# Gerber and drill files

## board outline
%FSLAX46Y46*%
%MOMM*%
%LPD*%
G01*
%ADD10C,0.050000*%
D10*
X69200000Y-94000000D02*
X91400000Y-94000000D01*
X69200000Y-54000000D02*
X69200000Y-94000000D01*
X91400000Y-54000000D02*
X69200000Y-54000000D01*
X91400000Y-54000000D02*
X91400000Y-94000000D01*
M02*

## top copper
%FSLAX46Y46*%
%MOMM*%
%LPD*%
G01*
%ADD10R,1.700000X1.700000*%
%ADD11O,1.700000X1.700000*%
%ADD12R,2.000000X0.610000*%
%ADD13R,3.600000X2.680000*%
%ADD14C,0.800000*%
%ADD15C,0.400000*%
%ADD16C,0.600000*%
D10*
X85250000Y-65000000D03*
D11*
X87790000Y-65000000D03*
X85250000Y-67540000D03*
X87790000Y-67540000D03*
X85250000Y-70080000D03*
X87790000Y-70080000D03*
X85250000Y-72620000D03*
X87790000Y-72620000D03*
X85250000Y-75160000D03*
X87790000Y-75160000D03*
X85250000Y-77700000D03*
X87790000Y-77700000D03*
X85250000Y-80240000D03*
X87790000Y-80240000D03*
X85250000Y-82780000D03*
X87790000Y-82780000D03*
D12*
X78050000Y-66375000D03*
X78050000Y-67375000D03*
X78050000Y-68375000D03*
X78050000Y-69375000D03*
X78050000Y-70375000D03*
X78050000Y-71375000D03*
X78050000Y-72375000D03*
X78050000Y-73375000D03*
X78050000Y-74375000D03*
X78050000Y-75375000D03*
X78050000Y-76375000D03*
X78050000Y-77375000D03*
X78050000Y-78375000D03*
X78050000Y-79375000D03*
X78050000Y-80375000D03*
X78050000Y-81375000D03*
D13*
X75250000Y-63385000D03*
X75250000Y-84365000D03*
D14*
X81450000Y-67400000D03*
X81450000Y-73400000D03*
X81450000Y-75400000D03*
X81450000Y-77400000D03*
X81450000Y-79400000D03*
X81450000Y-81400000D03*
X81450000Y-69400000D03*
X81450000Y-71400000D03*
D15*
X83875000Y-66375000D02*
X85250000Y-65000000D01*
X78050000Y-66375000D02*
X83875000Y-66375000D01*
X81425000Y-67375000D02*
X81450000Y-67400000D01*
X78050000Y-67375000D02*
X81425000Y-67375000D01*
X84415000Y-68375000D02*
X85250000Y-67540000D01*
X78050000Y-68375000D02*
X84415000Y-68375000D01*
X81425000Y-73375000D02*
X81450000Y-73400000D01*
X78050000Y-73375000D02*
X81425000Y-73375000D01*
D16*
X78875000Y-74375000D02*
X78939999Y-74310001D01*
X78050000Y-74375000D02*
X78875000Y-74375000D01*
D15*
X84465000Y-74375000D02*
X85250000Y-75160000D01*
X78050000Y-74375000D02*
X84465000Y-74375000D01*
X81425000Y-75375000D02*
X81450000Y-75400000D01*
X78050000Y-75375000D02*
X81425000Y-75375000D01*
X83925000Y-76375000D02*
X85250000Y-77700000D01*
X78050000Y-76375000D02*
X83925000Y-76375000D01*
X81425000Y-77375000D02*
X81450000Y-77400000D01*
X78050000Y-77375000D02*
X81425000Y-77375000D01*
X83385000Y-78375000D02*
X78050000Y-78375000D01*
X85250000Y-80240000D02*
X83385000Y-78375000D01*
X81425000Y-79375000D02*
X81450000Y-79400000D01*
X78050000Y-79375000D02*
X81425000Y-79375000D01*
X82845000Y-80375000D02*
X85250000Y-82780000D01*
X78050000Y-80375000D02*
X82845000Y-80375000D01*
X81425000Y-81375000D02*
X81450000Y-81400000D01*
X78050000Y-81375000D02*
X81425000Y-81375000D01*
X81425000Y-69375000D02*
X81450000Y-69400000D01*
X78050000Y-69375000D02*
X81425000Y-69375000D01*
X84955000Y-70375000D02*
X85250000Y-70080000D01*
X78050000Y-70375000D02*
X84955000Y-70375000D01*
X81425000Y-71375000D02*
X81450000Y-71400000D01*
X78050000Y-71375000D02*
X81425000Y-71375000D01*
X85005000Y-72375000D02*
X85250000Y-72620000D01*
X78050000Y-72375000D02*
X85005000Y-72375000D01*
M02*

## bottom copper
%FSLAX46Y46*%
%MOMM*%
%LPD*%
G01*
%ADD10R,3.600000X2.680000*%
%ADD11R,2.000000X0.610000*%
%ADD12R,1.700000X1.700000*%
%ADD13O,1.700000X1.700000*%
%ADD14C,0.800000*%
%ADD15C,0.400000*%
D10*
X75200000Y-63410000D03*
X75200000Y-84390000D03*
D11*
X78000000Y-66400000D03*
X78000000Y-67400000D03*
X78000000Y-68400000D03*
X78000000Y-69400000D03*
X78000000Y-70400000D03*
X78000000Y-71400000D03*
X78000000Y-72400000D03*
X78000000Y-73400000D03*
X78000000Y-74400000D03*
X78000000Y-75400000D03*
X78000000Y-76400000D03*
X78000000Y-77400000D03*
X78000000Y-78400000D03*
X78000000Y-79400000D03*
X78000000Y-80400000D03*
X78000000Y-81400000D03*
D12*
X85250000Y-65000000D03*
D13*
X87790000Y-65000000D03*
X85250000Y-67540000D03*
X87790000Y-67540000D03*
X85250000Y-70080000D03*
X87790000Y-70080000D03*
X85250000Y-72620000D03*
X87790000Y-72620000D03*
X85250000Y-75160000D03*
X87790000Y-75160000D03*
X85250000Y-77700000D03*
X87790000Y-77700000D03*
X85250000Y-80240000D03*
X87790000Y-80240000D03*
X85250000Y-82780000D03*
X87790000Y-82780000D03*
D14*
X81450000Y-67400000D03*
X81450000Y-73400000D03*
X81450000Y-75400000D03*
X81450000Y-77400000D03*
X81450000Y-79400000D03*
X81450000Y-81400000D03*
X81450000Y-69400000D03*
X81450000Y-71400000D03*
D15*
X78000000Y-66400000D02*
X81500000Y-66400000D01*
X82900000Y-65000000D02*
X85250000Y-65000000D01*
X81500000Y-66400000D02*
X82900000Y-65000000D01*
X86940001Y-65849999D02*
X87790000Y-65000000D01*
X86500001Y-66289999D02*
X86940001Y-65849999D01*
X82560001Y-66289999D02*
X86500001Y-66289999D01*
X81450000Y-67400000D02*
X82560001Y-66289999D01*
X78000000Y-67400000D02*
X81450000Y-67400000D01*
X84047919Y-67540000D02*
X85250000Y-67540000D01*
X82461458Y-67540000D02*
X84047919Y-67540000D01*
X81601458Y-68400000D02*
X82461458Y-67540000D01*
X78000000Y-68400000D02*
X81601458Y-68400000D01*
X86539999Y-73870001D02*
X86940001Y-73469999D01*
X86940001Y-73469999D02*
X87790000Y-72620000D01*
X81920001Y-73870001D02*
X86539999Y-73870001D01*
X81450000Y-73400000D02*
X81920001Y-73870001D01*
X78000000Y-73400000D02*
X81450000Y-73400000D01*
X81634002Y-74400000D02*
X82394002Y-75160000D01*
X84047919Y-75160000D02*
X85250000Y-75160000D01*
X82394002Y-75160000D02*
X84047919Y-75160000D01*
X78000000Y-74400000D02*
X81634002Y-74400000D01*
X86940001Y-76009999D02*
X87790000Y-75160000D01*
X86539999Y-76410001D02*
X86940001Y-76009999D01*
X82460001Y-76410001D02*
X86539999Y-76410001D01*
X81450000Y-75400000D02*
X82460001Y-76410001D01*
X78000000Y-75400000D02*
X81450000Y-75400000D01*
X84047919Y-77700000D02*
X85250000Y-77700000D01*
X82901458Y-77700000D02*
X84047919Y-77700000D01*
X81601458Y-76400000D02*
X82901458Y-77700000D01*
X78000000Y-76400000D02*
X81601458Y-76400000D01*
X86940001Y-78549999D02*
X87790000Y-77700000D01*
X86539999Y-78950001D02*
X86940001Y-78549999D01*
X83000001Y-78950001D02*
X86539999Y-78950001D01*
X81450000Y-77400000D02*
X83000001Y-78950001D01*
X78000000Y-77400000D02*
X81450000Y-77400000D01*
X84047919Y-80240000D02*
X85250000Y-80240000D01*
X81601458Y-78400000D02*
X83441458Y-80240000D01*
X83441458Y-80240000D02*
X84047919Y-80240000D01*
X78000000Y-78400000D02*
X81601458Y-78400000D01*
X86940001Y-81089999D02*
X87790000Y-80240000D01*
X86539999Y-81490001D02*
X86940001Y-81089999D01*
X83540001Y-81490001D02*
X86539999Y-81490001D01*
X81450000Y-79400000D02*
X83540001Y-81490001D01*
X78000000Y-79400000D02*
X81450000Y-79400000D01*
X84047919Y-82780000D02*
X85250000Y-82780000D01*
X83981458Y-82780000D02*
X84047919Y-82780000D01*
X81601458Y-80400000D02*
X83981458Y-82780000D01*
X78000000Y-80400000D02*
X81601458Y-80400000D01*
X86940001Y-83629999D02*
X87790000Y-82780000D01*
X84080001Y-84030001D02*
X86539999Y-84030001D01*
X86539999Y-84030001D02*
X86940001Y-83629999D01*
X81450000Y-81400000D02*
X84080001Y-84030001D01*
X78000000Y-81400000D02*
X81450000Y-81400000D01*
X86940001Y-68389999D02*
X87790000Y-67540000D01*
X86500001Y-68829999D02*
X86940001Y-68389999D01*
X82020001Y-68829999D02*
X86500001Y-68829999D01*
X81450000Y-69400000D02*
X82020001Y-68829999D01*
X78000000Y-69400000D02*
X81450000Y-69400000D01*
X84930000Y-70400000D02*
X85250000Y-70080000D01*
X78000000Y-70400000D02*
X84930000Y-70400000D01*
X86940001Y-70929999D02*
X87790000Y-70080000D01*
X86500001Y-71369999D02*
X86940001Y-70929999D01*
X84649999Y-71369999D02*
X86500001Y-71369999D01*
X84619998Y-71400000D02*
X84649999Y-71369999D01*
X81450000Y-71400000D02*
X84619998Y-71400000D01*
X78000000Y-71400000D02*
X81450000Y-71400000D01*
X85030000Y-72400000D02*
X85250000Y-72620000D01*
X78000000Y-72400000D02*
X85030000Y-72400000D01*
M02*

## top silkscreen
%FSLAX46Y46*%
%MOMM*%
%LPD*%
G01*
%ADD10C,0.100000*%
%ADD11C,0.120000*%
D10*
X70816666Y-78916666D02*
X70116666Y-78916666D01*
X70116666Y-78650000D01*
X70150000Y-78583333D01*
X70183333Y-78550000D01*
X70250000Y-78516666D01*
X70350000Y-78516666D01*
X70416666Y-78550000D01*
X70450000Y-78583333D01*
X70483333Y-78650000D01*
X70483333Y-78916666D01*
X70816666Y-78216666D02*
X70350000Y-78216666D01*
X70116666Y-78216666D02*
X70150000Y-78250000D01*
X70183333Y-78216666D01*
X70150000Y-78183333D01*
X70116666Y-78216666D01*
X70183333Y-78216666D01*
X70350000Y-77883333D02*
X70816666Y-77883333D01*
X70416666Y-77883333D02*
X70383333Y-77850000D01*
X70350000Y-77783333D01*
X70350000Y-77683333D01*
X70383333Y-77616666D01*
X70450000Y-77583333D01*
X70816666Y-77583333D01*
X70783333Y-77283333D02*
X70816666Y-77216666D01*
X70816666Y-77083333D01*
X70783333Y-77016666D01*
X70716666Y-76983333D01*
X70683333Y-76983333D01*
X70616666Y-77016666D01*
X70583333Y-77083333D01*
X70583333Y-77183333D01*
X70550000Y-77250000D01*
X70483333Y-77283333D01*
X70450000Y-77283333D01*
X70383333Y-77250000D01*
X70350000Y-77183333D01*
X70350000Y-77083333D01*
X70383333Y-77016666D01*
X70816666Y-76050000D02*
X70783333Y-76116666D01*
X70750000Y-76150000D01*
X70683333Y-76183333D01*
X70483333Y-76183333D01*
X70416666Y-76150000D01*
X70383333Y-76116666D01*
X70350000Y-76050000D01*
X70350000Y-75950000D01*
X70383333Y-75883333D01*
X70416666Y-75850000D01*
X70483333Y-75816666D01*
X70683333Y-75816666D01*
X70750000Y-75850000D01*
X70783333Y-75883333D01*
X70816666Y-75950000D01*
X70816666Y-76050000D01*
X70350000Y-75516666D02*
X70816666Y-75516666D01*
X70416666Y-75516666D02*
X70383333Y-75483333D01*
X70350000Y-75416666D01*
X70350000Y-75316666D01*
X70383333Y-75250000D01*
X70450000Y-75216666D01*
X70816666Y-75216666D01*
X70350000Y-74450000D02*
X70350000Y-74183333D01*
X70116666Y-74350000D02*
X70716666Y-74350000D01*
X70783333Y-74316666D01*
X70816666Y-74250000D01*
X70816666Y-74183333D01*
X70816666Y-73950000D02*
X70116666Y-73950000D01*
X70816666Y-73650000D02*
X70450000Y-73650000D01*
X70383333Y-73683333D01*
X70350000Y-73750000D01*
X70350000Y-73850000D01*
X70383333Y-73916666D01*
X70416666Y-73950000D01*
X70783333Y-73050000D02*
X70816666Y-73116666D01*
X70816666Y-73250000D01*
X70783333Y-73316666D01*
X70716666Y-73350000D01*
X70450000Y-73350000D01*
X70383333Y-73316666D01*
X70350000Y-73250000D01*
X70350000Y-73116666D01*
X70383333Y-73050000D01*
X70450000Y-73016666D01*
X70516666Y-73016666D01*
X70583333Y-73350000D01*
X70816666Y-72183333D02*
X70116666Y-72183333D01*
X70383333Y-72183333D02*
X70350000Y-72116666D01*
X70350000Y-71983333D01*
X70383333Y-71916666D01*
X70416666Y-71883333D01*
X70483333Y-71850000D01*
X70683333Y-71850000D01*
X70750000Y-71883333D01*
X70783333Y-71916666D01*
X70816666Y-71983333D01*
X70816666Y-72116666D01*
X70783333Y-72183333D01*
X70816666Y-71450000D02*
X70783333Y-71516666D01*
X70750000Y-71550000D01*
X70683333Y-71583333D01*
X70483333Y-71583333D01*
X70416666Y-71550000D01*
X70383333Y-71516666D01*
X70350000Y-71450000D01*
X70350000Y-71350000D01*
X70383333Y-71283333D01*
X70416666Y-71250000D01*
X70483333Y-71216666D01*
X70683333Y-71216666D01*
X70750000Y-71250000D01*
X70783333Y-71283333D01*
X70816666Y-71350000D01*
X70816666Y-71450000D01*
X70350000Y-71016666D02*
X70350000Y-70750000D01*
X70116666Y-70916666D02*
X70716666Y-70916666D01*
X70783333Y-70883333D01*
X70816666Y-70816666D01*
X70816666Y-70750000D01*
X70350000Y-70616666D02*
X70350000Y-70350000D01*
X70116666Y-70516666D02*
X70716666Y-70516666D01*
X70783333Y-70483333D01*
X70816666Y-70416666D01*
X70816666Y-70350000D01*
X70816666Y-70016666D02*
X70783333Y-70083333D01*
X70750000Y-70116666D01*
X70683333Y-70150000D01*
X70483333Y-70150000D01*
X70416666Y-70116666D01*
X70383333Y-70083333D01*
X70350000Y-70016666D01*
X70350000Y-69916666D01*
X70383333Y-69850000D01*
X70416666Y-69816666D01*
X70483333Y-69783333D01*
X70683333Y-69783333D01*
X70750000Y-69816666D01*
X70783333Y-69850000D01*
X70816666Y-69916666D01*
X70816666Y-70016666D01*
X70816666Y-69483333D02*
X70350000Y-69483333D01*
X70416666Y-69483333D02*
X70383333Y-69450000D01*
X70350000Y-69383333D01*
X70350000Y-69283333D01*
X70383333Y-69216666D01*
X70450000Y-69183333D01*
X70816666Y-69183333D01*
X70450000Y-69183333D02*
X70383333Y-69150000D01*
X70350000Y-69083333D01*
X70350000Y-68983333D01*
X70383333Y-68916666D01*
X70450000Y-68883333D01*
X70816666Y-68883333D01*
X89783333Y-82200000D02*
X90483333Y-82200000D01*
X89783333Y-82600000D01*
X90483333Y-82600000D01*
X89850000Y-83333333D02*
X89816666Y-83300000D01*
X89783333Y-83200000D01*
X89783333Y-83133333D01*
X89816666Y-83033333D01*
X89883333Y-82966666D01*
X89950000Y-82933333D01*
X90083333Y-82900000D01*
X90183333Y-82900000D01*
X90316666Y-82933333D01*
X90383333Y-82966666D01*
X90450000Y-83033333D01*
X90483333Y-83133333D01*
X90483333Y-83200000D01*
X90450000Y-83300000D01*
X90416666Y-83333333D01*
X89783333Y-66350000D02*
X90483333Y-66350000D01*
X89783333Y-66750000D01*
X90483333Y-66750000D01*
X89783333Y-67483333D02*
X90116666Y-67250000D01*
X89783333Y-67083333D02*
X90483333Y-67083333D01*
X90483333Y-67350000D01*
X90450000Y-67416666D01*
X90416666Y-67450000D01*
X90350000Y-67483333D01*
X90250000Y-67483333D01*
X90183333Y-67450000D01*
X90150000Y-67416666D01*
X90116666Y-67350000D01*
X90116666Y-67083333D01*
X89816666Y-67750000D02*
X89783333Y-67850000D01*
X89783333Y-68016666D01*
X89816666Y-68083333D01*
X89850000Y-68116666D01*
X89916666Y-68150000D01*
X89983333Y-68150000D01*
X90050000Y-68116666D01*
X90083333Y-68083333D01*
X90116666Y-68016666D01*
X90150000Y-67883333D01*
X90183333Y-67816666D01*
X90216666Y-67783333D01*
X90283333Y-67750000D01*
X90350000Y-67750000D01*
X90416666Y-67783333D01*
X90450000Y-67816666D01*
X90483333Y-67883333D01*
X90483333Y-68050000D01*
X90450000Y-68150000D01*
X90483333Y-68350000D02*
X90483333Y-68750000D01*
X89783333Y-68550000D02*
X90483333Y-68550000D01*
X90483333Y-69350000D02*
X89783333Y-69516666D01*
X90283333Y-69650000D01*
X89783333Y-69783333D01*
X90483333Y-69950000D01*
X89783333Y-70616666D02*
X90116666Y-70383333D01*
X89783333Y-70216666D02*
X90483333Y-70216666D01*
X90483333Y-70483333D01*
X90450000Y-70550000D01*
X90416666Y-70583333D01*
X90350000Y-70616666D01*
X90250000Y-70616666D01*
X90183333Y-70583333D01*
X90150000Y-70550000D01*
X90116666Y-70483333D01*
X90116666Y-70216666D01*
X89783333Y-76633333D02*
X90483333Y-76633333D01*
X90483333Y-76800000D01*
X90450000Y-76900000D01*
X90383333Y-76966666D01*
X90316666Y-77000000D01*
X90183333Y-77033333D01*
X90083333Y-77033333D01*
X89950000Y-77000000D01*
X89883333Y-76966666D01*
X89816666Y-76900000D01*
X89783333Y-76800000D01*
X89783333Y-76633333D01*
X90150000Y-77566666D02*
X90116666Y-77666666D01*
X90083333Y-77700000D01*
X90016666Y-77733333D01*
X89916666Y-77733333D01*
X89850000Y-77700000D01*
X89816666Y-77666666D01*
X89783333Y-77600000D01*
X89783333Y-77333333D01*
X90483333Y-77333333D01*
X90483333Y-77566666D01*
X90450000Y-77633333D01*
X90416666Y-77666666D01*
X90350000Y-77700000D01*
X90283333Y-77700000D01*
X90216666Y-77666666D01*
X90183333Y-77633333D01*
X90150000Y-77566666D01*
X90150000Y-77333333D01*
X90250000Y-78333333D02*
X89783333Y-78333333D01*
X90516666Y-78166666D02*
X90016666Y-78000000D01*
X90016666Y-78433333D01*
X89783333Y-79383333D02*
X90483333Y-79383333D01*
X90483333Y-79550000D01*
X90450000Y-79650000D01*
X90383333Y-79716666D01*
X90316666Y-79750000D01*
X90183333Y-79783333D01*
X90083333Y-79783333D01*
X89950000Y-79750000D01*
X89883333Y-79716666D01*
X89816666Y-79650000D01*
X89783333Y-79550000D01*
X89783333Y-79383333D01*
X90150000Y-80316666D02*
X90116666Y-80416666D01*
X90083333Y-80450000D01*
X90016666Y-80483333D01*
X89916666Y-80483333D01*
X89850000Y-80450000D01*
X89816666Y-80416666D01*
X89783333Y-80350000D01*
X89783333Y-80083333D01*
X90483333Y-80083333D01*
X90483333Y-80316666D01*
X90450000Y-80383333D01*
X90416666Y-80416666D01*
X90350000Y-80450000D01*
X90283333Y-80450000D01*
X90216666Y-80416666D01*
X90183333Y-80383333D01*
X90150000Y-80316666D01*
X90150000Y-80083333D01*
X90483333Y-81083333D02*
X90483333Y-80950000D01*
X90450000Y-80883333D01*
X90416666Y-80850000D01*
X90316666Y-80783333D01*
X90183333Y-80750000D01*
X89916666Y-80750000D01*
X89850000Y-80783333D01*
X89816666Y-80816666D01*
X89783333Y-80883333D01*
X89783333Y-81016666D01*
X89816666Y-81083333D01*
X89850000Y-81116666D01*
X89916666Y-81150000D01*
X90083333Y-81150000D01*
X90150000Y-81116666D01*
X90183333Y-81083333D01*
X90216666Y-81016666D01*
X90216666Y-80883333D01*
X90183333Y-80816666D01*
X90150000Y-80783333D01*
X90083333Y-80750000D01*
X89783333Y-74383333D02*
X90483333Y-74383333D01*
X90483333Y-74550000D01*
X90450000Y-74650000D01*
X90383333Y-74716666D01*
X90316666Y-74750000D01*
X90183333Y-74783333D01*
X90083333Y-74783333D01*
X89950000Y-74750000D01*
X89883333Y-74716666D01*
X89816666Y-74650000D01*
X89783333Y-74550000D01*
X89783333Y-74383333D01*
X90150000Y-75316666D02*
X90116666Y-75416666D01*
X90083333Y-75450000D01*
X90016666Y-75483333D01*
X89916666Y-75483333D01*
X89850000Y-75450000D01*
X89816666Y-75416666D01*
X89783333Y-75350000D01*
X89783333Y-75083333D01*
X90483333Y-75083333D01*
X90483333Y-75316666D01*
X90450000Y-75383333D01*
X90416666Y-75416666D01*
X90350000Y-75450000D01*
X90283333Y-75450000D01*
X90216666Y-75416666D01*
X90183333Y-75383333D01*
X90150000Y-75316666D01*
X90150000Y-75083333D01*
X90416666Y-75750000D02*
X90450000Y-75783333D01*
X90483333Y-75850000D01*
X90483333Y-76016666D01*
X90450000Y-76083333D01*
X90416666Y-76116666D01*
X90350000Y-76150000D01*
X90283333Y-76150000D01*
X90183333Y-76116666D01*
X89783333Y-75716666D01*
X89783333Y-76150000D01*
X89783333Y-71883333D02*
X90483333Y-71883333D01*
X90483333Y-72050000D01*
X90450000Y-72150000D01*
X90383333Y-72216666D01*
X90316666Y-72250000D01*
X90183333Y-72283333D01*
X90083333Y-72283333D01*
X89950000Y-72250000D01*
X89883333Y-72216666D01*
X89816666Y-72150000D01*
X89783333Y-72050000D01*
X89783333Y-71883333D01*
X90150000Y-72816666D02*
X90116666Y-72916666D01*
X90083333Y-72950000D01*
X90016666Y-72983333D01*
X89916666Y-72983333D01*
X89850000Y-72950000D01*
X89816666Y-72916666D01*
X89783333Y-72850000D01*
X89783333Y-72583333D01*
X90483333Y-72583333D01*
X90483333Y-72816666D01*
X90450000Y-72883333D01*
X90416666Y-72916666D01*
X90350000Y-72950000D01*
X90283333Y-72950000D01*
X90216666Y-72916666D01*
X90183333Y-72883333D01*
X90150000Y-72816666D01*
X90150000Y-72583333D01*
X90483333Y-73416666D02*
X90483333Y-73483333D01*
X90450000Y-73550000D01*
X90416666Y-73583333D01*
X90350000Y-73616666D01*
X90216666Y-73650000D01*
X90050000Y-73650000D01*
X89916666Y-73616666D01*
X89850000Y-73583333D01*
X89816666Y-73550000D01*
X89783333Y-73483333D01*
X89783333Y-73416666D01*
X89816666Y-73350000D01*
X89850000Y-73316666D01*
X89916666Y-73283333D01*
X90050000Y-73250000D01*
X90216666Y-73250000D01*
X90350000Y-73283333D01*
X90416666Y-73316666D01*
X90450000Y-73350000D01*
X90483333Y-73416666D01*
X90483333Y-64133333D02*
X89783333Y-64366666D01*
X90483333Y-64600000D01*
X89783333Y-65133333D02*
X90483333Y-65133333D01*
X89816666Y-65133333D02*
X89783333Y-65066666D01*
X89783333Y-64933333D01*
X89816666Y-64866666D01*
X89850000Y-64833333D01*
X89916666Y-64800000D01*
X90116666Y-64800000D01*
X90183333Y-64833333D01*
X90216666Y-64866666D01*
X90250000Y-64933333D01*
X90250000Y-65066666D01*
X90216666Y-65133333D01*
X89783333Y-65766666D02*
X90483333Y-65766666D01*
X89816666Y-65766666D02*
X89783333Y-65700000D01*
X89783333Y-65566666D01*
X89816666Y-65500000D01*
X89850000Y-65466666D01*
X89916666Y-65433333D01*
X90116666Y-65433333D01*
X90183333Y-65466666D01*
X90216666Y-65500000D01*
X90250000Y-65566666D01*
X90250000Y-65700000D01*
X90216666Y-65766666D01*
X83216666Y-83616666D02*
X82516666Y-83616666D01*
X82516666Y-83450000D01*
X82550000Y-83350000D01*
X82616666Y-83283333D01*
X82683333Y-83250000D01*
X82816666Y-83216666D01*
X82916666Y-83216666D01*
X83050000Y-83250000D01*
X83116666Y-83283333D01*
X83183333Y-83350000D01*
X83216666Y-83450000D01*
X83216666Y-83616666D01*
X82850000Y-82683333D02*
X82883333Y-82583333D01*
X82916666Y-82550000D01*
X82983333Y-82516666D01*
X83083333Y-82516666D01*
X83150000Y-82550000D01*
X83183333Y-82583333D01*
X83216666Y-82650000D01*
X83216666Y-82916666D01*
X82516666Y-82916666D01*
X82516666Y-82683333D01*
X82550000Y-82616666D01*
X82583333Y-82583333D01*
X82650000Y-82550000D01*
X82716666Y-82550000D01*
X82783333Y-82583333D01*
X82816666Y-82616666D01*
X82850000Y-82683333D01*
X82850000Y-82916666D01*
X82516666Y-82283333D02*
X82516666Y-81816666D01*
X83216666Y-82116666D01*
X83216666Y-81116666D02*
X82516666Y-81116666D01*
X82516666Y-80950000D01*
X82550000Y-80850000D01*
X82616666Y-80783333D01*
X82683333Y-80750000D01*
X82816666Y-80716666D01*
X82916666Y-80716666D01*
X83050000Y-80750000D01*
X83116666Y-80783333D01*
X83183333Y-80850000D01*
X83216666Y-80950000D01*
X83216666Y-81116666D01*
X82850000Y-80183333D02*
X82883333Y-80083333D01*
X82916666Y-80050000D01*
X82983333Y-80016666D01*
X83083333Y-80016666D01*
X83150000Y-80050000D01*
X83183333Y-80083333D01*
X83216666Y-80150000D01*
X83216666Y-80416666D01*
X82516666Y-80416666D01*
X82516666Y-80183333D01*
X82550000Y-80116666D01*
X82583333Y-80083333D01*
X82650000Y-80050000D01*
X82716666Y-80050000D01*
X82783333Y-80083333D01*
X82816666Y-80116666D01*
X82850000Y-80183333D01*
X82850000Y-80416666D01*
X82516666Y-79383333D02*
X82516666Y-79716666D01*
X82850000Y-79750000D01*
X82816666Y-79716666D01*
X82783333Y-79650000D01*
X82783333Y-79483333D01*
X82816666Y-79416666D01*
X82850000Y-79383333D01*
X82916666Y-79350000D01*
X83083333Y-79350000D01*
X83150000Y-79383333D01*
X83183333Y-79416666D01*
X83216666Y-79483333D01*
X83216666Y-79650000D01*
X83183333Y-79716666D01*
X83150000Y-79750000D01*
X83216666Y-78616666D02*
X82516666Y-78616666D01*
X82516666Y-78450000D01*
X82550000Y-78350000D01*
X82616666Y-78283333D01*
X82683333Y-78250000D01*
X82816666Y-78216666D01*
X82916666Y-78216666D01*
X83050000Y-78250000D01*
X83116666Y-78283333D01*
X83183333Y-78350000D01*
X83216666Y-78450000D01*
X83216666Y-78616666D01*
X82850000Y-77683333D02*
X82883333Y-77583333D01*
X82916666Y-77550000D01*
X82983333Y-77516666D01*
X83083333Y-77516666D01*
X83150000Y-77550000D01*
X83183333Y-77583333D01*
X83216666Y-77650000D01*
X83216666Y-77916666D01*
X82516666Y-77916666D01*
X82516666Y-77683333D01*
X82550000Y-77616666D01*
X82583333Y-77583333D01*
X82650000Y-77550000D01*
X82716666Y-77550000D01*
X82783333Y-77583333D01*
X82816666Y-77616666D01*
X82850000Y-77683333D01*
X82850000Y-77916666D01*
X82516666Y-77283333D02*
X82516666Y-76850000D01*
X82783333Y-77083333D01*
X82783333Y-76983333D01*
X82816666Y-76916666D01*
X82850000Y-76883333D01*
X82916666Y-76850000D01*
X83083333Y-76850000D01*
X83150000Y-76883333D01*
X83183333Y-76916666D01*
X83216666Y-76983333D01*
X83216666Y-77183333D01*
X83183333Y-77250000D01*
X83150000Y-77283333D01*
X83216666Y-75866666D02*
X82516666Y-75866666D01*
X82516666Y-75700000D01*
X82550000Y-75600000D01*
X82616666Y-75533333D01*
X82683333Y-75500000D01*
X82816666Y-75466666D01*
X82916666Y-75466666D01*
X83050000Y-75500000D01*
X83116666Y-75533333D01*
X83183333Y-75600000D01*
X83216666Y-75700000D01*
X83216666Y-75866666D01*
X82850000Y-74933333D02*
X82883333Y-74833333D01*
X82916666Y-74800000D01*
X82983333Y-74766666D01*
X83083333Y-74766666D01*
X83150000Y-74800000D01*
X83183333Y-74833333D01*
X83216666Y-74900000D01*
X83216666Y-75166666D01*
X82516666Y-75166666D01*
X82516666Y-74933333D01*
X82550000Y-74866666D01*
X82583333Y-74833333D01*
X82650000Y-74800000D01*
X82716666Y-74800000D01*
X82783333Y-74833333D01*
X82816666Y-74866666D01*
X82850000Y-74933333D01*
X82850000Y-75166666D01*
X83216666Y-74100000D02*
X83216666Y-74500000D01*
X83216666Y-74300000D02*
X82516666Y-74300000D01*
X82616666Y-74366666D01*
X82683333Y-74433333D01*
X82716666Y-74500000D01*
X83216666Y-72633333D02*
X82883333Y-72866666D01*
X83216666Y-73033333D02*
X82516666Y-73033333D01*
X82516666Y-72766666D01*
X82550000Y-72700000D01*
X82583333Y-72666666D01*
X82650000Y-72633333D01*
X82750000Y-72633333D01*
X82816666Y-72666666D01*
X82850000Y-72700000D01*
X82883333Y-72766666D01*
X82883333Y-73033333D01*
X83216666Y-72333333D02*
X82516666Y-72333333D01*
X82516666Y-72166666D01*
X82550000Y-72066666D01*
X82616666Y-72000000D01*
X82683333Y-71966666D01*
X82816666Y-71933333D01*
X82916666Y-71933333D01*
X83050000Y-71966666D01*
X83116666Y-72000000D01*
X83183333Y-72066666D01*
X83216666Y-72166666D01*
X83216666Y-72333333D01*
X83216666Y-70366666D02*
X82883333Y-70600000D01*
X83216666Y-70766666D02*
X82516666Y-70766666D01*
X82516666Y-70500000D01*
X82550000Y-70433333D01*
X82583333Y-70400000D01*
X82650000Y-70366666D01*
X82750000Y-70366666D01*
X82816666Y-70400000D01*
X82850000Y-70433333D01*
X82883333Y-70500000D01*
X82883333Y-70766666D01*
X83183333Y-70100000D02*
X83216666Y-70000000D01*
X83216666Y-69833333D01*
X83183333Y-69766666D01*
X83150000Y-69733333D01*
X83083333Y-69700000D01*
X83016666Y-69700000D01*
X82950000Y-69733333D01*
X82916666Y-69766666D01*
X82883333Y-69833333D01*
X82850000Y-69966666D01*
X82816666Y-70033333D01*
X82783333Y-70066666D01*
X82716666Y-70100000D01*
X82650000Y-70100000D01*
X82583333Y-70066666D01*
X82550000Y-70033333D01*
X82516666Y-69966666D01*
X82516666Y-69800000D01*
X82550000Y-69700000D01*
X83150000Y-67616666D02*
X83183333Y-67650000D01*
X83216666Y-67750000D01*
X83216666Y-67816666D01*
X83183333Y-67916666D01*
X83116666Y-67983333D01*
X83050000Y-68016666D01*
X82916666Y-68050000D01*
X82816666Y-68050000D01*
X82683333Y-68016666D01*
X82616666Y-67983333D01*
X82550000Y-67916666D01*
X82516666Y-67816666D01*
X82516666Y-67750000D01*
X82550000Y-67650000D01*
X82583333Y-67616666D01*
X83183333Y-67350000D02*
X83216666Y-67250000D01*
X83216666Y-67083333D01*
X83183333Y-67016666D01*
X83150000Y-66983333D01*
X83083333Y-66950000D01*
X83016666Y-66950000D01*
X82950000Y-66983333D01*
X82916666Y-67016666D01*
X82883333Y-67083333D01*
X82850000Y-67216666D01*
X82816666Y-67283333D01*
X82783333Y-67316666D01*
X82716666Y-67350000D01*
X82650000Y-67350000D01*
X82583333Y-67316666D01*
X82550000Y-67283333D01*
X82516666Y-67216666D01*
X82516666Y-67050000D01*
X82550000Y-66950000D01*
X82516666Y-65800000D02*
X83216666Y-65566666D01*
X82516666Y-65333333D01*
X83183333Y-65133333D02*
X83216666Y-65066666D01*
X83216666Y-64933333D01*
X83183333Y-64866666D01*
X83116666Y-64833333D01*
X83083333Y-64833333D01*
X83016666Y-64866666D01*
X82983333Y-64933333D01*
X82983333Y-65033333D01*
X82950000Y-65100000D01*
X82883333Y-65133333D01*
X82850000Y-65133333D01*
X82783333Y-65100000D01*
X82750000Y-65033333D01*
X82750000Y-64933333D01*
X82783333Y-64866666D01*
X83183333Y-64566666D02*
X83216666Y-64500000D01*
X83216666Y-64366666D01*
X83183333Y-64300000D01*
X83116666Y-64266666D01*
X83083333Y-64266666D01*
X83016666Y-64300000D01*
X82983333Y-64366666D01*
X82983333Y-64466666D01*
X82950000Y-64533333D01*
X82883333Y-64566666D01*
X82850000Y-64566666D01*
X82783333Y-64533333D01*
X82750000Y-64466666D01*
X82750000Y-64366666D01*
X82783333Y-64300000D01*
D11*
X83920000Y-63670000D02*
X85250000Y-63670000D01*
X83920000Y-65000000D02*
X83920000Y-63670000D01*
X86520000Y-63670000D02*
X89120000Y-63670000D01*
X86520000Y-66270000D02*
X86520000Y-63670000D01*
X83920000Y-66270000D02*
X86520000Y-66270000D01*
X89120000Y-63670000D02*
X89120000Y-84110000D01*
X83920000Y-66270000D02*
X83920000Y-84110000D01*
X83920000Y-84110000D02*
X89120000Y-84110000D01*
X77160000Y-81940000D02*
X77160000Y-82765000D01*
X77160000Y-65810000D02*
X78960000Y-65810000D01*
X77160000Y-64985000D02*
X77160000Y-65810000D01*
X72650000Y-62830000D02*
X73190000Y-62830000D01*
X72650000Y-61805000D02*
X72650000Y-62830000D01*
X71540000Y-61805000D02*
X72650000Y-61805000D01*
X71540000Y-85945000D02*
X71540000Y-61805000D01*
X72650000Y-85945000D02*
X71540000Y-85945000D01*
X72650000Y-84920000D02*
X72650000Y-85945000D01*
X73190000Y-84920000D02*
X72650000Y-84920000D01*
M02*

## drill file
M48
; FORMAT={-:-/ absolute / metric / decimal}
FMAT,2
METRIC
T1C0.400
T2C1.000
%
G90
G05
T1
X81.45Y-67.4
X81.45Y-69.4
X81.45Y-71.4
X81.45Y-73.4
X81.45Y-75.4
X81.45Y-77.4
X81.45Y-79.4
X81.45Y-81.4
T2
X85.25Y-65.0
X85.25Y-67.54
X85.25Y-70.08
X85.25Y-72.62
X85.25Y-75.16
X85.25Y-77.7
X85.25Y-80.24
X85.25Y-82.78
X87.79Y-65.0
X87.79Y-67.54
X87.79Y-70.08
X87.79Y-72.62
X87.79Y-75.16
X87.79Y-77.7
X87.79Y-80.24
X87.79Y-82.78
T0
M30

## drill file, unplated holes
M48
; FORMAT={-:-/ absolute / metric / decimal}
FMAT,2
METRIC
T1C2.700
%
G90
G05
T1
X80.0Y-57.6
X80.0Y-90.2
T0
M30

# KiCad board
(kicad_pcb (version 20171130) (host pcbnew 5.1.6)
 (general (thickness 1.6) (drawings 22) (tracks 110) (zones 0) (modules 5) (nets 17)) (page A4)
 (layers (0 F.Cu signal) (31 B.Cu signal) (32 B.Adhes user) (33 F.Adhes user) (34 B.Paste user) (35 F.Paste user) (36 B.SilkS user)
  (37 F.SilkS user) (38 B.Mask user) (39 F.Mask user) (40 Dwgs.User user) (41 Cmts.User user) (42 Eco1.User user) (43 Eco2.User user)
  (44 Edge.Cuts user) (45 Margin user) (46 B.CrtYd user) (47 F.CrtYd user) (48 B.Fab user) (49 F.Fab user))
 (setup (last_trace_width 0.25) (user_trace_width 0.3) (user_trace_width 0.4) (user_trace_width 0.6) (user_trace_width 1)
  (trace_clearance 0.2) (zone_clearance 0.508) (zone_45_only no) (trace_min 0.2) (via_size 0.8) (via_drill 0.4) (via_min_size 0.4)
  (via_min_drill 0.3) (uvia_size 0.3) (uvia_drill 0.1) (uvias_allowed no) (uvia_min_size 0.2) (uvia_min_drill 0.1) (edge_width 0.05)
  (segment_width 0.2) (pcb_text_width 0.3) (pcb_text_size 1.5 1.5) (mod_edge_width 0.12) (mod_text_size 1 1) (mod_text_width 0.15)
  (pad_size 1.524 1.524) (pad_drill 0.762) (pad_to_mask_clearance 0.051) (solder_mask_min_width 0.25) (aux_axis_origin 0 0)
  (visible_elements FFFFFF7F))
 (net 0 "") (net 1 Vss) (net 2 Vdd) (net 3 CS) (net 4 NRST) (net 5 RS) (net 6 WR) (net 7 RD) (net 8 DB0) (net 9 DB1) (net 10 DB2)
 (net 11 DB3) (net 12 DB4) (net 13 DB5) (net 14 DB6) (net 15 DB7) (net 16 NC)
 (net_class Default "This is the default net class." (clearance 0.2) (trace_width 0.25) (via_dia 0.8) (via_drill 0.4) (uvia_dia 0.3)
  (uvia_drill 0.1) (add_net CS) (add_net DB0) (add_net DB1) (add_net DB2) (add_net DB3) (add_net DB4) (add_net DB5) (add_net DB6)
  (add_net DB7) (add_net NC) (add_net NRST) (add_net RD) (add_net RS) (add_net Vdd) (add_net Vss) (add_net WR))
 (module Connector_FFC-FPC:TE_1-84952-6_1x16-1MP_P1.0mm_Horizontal (layer B.Cu) (at 76.2 73.9 90)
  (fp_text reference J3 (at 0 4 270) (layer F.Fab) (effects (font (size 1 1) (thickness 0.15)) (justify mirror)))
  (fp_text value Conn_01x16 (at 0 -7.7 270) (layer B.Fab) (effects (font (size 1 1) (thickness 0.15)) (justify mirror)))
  (pad MP smd rect (at 10.49 -1 90) (size 2.68 3.6) (layers B.Cu B.Paste B.Mask))
  (pad MP smd rect (at -10.49 -1 90) (size 2.68 3.6) (layers B.Cu B.Paste B.Mask))
  (pad 16 smd rect (at 7.5 1.8 90) (size 0.61 2) (layers B.Cu B.Paste B.Mask) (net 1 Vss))
  (pad 15 smd rect (at 6.5 1.8 90) (size 0.61 2) (layers B.Cu B.Paste B.Mask) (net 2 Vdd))
  (pad 14 smd rect (at 5.5 1.8 90) (size 0.61 2) (layers B.Cu B.Paste B.Mask) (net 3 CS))
  (pad 13 smd rect (at 4.5 1.8 90) (size 0.61 2) (layers B.Cu B.Paste B.Mask) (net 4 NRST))
  (pad 12 smd rect (at 3.5 1.8 90) (size 0.61 2) (layers B.Cu B.Paste B.Mask) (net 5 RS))
  (pad 11 smd rect (at 2.5 1.8 90) (size 0.61 2) (layers B.Cu B.Paste B.Mask) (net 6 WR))
  (pad 10 smd rect (at 1.5 1.8 90) (size 0.61 2) (layers B.Cu B.Paste B.Mask) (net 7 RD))
  (pad 9 smd rect (at 0.5 1.8 90) (size 0.61 2) (layers B.Cu B.Paste B.Mask) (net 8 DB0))
  (pad 8 smd rect (at -0.5 1.8 90) (size 0.61 2) (layers B.Cu B.Paste B.Mask) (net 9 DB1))
  (pad 7 smd rect (at -1.5 1.8 90) (size 0.61 2) (layers B.Cu B.Paste B.Mask) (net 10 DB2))
  (pad 6 smd rect (at -2.5 1.8 90) (size 0.61 2) (layers B.Cu B.Paste B.Mask) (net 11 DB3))
  (pad 5 smd rect (at -3.5 1.8 90) (size 0.61 2) (layers B.Cu B.Paste B.Mask) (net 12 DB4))
  (pad 4 smd rect (at -4.5 1.8 90) (size 0.61 2) (layers B.Cu B.Paste B.Mask) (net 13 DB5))
  (pad 3 smd rect (at -5.5 1.8 90) (size 0.61 2) (layers B.Cu B.Paste B.Mask) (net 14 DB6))
  (pad 2 smd rect (at -6.5 1.8 90) (size 0.61 2) (layers B.Cu B.Paste B.Mask) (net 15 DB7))
  (pad 1 smd rect (at -7.5 1.8 90) (size 0.61 2) (layers B.Cu B.Paste B.Mask) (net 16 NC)))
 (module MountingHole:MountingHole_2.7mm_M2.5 (layer F.Cu) (at 80 90.2)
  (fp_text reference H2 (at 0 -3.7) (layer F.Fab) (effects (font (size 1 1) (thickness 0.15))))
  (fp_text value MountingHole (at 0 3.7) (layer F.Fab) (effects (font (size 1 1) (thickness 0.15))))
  (pad 1 np_thru_hole circle (at 0 0) (size 2.7 2.7) (drill 2.7) (layers *.Cu *.Mask)))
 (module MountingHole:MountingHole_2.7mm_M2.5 (layer F.Cu) (at 80 57.6)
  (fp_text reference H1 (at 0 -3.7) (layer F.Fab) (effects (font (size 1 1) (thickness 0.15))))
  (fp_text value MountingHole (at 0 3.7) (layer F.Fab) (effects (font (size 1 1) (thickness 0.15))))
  (pad 1 np_thru_hole circle (at 0 0) (size 2.7 2.7) (drill 2.7) (layers *.Cu *.Mask)))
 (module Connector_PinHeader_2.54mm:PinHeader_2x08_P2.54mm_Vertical (layer F.Cu) (at 85.25 65)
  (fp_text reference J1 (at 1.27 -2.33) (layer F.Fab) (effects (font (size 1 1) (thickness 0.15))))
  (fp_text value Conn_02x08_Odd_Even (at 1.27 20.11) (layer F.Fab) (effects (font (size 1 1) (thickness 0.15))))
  (fp_line (start -1.33 -1.33) (end 0 -1.33) (layer F.SilkS) (width 0.12))
  (fp_line (start -1.33 0) (end -1.33 -1.33) (layer F.SilkS) (width 0.12))
  (fp_line (start 1.27 -1.33) (end 3.87 -1.33) (layer F.SilkS) (width 0.12))
  (fp_line (start 1.27 1.27) (end 1.27 -1.33) (layer F.SilkS) (width 0.12))
  (fp_line (start -1.33 1.27) (end 1.27 1.27) (layer F.SilkS) (width 0.12))
  (fp_line (start 3.87 -1.33) (end 3.87 19.11) (layer F.SilkS) (width 0.12))
  (fp_line (start -1.33 1.27) (end -1.33 19.11) (layer F.SilkS) (width 0.12))
  (fp_line (start -1.33 19.11) (end 3.87 19.11) (layer F.SilkS) (width 0.12))
  (pad 1 thru_hole rect (at 0 0) (size 1.7 1.7) (drill 1) (layers *.Cu *.Mask) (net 1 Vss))
  (pad 2 thru_hole oval (at 2.54 0) (size 1.7 1.7) (drill 1) (layers *.Cu *.Mask) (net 2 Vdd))
  (pad 3 thru_hole oval (at 0 2.54) (size 1.7 1.7) (drill 1) (layers *.Cu *.Mask) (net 3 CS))
  (pad 4 thru_hole oval (at 2.54 2.54) (size 1.7 1.7) (drill 1) (layers *.Cu *.Mask) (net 4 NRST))
  (pad 5 thru_hole oval (at 0 5.08) (size 1.7 1.7) (drill 1) (layers *.Cu *.Mask) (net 5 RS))
  (pad 6 thru_hole oval (at 2.54 5.08) (size 1.7 1.7) (drill 1) (layers *.Cu *.Mask) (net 6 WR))
  (pad 7 thru_hole oval (at 0 7.62) (size 1.7 1.7) (drill 1) (layers *.Cu *.Mask) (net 7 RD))
  (pad 8 thru_hole oval (at 2.54 7.62) (size 1.7 1.7) (drill 1) (layers *.Cu *.Mask) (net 8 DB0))
  (pad 9 thru_hole oval (at 0 10.16) (size 1.7 1.7) (drill 1) (layers *.Cu *.Mask) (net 9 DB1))
  (pad 10 thru_hole oval (at 2.54 10.16) (size 1.7 1.7) (drill 1) (layers *.Cu *.Mask) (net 10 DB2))
  (pad 11 thru_hole oval (at 0 12.7) (size 1.7 1.7) (drill 1) (layers *.Cu *.Mask) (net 11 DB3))
  (pad 12 thru_hole oval (at 2.54 12.7) (size 1.7 1.7) (drill 1) (layers *.Cu *.Mask) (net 12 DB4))
  (pad 13 thru_hole oval (at 0 15.24) (size 1.7 1.7) (drill 1) (layers *.Cu *.Mask) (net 13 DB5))
  (pad 14 thru_hole oval (at 2.54 15.24) (size 1.7 1.7) (drill 1) (layers *.Cu *.Mask) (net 14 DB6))
  (pad 15 thru_hole oval (at 0 17.78) (size 1.7 1.7) (drill 1) (layers *.Cu *.Mask) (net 15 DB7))
  (pad 16 thru_hole oval (at 2.54 17.78) (size 1.7 1.7) (drill 1) (layers *.Cu *.Mask) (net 16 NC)))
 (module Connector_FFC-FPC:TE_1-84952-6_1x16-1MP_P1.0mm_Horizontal (layer F.Cu) (at 76.25 73.875 270)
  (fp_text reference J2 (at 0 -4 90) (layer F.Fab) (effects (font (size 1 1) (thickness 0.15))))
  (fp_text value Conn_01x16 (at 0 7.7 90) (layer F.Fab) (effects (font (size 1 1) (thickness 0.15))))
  (fp_line (start 8.065 -0.91) (end 8.89 -0.91) (layer F.SilkS) (width 0.12))
  (fp_line (start -8.065 -0.91) (end -8.065 -2.71) (layer F.SilkS) (width 0.12))
  (fp_line (start -8.89 -0.91) (end -8.065 -0.91) (layer F.SilkS) (width 0.12))
  (fp_line (start -11.045 3.6) (end -11.045 3.06) (layer F.SilkS) (width 0.12))
  (fp_line (start -12.07 3.6) (end -11.045 3.6) (layer F.SilkS) (width 0.12))
  (fp_line (start -12.07 4.71) (end -12.07 3.6) (layer F.SilkS) (width 0.12))
  (fp_line (start 12.07 4.71) (end -12.07 4.71) (layer F.SilkS) (width 0.12))
  (fp_line (start 12.07 3.6) (end 12.07 4.71) (layer F.SilkS) (width 0.12))
  (fp_line (start 11.045 3.6) (end 12.07 3.6) (layer F.SilkS) (width 0.12))
  (fp_line (start 11.045 3.06) (end 11.045 3.6) (layer F.SilkS) (width 0.12))
  (pad 1 smd rect (at -7.5 -1.8 270) (size 0.61 2) (layers F.Cu F.Paste F.Mask) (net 1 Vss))
  (pad 2 smd rect (at -6.5 -1.8 270) (size 0.61 2) (layers F.Cu F.Paste F.Mask) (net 2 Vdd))
  (pad 3 smd rect (at -5.5 -1.8 270) (size 0.61 2) (layers F.Cu F.Paste F.Mask) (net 3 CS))
  (pad 4 smd rect (at -4.5 -1.8 270) (size 0.61 2) (layers F.Cu F.Paste F.Mask) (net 4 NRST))
  (pad 5 smd rect (at -3.5 -1.8 270) (size 0.61 2) (layers F.Cu F.Paste F.Mask) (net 5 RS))
  (pad 6 smd rect (at -2.5 -1.8 270) (size 0.61 2) (layers F.Cu F.Paste F.Mask) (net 6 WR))
  (pad 7 smd rect (at -1.5 -1.8 270) (size 0.61 2) (layers F.Cu F.Paste F.Mask) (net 7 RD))
  (pad 8 smd rect (at -0.5 -1.8 270) (size 0.61 2) (layers F.Cu F.Paste F.Mask) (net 8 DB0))
  (pad 9 smd rect (at 0.5 -1.8 270) (size 0.61 2) (layers F.Cu F.Paste F.Mask) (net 9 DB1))
  (pad 10 smd rect (at 1.5 -1.8 270) (size 0.61 2) (layers F.Cu F.Paste F.Mask) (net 10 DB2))
  (pad 11 smd rect (at 2.5 -1.8 270) (size 0.61 2) (layers F.Cu F.Paste F.Mask) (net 11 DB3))
  (pad 12 smd rect (at 3.5 -1.8 270) (size 0.61 2) (layers F.Cu F.Paste F.Mask) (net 12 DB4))
  (pad 13 smd rect (at 4.5 -1.8 270) (size 0.61 2) (layers F.Cu F.Paste F.Mask) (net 13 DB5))
  (pad 14 smd rect (at 5.5 -1.8 270) (size 0.61 2) (layers F.Cu F.Paste F.Mask) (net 14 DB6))
  (pad 15 smd rect (at 6.5 -1.8 270) (size 0.61 2) (layers F.Cu F.Paste F.Mask) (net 15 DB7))
  (pad 16 smd rect (at 7.5 -1.8 270) (size 0.61 2) (layers F.Cu F.Paste F.Mask) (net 16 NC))
  (pad MP smd rect (at -10.49 1 270) (size 2.68 3.6) (layers F.Cu F.Paste F.Mask))
  (pad MP smd rect (at 10.49 1 270) (size 2.68 3.6) (layers F.Cu F.Paste F.Mask)))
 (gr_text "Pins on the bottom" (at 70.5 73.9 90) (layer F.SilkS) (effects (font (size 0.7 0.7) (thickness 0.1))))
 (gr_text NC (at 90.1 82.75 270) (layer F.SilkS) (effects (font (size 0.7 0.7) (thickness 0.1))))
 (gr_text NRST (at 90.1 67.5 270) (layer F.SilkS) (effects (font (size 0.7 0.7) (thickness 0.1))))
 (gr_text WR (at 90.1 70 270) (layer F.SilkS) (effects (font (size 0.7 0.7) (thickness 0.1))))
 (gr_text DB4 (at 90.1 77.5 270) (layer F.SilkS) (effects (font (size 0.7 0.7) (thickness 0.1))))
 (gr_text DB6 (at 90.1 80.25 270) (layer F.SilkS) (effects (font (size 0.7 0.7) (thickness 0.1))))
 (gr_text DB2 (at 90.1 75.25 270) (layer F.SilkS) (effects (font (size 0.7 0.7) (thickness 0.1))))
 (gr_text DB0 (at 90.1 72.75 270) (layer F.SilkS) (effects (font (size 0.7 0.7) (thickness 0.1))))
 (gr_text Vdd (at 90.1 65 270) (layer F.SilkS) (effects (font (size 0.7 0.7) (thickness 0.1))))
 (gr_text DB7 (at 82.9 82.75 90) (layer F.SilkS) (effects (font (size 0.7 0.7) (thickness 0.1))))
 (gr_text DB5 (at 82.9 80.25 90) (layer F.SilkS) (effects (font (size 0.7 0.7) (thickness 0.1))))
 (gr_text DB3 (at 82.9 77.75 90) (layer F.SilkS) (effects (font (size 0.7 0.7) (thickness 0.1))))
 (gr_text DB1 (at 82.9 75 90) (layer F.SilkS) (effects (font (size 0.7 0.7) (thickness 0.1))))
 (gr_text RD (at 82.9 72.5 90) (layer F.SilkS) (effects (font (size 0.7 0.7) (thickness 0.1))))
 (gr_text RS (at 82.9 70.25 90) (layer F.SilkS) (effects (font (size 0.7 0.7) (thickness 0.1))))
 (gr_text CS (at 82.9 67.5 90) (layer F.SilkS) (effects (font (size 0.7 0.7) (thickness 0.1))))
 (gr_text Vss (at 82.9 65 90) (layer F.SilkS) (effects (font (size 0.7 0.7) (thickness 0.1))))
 (gr_line (start 69.2 94) (end 91.4 94) (layer Edge.Cuts) (width 0.05))
 (gr_line (start 69.2 54) (end 69.2 94) (layer Edge.Cuts) (width 0.05))
 (gr_line (start 91.4 54) (end 69.2 54) (layer Edge.Cuts) (width 0.05))
 (gr_line (start 91.4 54) (end 91.4 94) (layer Edge.Cuts) (width 0.05))
 (segment (start 83.875 66.375) (end 85.25 65) (width 0.4) (layer F.Cu) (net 1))
 (segment (start 78.05 66.375) (end 83.875 66.375) (width 0.4) (layer F.Cu) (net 1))
 (segment (start 78 66.4) (end 81.5 66.4) (width 0.4) (layer B.Cu) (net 1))
 (segment (start 82.9 65) (end 85.25 65) (width 0.4) (layer B.Cu) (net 1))
 (segment (start 81.5 66.4) (end 82.9 65) (width 0.4) (layer B.Cu) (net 1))
 (via (at 81.45 67.4) (size 0.8) (drill 0.4) (layers F.Cu B.Cu) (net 2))
 (segment (start 86.940001 65.849999) (end 87.79 65) (width 0.4) (layer B.Cu) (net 2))
 (segment (start 86.500001 66.289999) (end 86.940001 65.849999) (width 0.4) (layer B.Cu) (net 2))
 (segment (start 82.560001 66.289999) (end 86.500001 66.289999) (width 0.4) (layer B.Cu) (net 2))
 (segment (start 81.45 67.4) (end 82.560001 66.289999) (width 0.4) (layer B.Cu) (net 2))
 (segment (start 81.425 67.375) (end 81.45 67.4) (width 0.4) (layer F.Cu) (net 2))
 (segment (start 78.05 67.375) (end 81.425 67.375) (width 0.4) (layer F.Cu) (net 2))
 (segment (start 78 67.4) (end 81.45 67.4) (width 0.4) (layer B.Cu) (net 2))
 (segment (start 84.415 68.375) (end 85.25 67.54) (width 0.4) (layer F.Cu) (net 3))
 (segment (start 78.05 68.375) (end 84.415 68.375) (width 0.4) (layer F.Cu) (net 3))
 (segment (start 84.047919 67.54) (end 85.25 67.54) (width 0.4) (layer B.Cu) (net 3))
 (segment (start 82.461458 67.54) (end 84.047919 67.54) (width 0.4) (layer B.Cu) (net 3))
 (segment (start 81.601458 68.4) (end 82.461458 67.54) (width 0.4) (layer B.Cu) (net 3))
 (segment (start 78 68.4) (end 81.601458 68.4) (width 0.4) (layer B.Cu) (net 3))
 (via (at 81.45 73.4) (size 0.8) (drill 0.4) (layers F.Cu B.Cu) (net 8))
 (segment (start 86.539999 73.870001) (end 86.940001 73.469999) (width 0.4) (layer B.Cu) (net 8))
 (segment (start 86.940001 73.469999) (end 87.79 72.62) (width 0.4) (layer B.Cu) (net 8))
 (segment (start 81.920001 73.870001) (end 86.539999 73.870001) (width 0.4) (layer B.Cu) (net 8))
 (segment (start 81.45 73.4) (end 81.920001 73.870001) (width 0.4) (layer B.Cu) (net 8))
 (segment (start 81.425 73.375) (end 81.45 73.4) (width 0.4) (layer F.Cu) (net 8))
 (segment (start 78.05 73.375) (end 81.425 73.375) (width 0.4) (layer F.Cu) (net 8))
 (segment (start 78 73.4) (end 81.45 73.4) (width 0.4) (layer B.Cu) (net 8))
 (segment (start 78.875 74.375) (end 78.939999 74.310001) (width 0.6) (layer F.Cu) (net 9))
 (segment (start 78.05 74.375) (end 78.875 74.375) (width 0.6) (layer F.Cu) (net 9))
 (segment (start 84.465 74.375) (end 85.25 75.16) (width 0.4) (layer F.Cu) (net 9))
 (segment (start 78.05 74.375) (end 84.465 74.375) (width 0.4) (layer F.Cu) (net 9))
 (segment (start 81.634002 74.4) (end 82.394002 75.16) (width 0.4) (layer B.Cu) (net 9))
 (segment (start 84.047919 75.16) (end 85.25 75.16) (width 0.4) (layer B.Cu) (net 9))
 (segment (start 82.394002 75.16) (end 84.047919 75.16) (width 0.4) (layer B.Cu) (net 9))
 (segment (start 78 74.4) (end 81.634002 74.4) (width 0.4) (layer B.Cu) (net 9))
 (via (at 81.45 75.4) (size 0.8) (drill 0.4) (layers F.Cu B.Cu) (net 10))
 (segment (start 86.940001 76.009999) (end 87.79 75.16) (width 0.4) (layer B.Cu) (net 10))
 (segment (start 86.539999 76.410001) (end 86.940001 76.009999) (width 0.4) (layer B.Cu) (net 10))
 (segment (start 82.460001 76.410001) (end 86.539999 76.410001) (width 0.4) (layer B.Cu) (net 10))
 (segment (start 81.45 75.4) (end 82.460001 76.410001) (width 0.4) (layer B.Cu) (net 10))
 (segment (start 81.425 75.375) (end 81.45 75.4) (width 0.4) (layer F.Cu) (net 10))
 (segment (start 78.05 75.375) (end 81.425 75.375) (width 0.4) (layer F.Cu) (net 10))
 (segment (start 78 75.4) (end 81.45 75.4) (width 0.4) (layer B.Cu) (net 10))
 (segment (start 83.925 76.375) (end 85.25 77.7) (width 0.4) (layer F.Cu) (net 11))
 (segment (start 78.05 76.375) (end 83.925 76.375) (width 0.4) (layer F.Cu) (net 11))
 (segment (start 84.047919 77.7) (end 85.25 77.7) (width 0.4) (layer B.Cu) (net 11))
 (segment (start 82.901458 77.7) (end 84.047919 77.7) (width 0.4) (layer B.Cu) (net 11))
 (segment (start 81.601458 76.4) (end 82.901458 77.7) (width 0.4) (layer B.Cu) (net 11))
 (segment (start 78 76.4) (end 81.601458 76.4) (width 0.4) (layer B.Cu) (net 11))
 (via (at 81.45 77.4) (size 0.8) (drill 0.4) (layers F.Cu B.Cu) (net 12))
 (segment (start 86.940001 78.549999) (end 87.79 77.7) (width 0.4) (layer B.Cu) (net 12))
 (segment (start 86.539999 78.950001) (end 86.940001 78.549999) (width 0.4) (layer B.Cu) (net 12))
 (segment (start 83.000001 78.950001) (end 86.539999 78.950001) (width 0.4) (layer B.Cu) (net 12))
 (segment (start 81.45 77.4) (end 83.000001 78.950001) (width 0.4) (layer B.Cu) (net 12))
 (segment (start 81.425 77.375) (end 81.45 77.4) (width 0.4) (layer F.Cu) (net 12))
 (segment (start 78.05 77.375) (end 81.425 77.375) (width 0.4) (layer F.Cu) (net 12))
 (segment (start 78 77.4) (end 81.45 77.4) (width 0.4) (layer B.Cu) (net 12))
 (segment (start 84.047919 80.24) (end 85.25 80.24) (width 0.4) (layer B.Cu) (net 13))
 (segment (start 81.601458 78.4) (end 83.441458 80.24) (width 0.4) (layer B.Cu) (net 13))
 (segment (start 83.441458 80.24) (end 84.047919 80.24) (width 0.4) (layer B.Cu) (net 13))
 (segment (start 78 78.4) (end 81.601458 78.4) (width 0.4) (layer B.Cu) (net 13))
 (segment (start 83.385 78.375) (end 78.05 78.375) (width 0.4) (layer F.Cu) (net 13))
 (segment (start 85.25 80.24) (end 83.385 78.375) (width 0.4) (layer F.Cu) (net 13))
 (via (at 81.45 79.4) (size 0.8) (drill 0.4) (layers F.Cu B.Cu) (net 14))
 (segment (start 86.940001 81.089999) (end 87.79 80.24) (width 0.4) (layer B.Cu) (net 14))
 (segment (start 86.539999 81.490001) (end 86.940001 81.089999) (width 0.4) (layer B.Cu) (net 14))
 (segment (start 83.540001 81.490001) (end 86.539999 81.490001) (width 0.4) (layer B.Cu) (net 14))
 (segment (start 81.45 79.4) (end 83.540001 81.490001) (width 0.4) (layer B.Cu) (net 14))
 (segment (start 81.425 79.375) (end 81.45 79.4) (width 0.4) (layer F.Cu) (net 14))
 (segment (start 78.05 79.375) (end 81.425 79.375) (width 0.4) (layer F.Cu) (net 14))
 (segment (start 78 79.4) (end 81.45 79.4) (width 0.4) (layer B.Cu) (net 14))
 (segment (start 82.845 80.375) (end 85.25 82.78) (width 0.4) (layer F.Cu) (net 15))
 (segment (start 78.05 80.375) (end 82.845 80.375) (width 0.4) (layer F.Cu) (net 15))
 (segment (start 84.047919 82.78) (end 85.25 82.78) (width 0.4) (layer B.Cu) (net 15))
 (segment (start 83.981458 82.78) (end 84.047919 82.78) (width 0.4) (layer B.Cu) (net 15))
 (segment (start 81.601458 80.4) (end 83.981458 82.78) (width 0.4) (layer B.Cu) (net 15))
 (segment (start 78 80.4) (end 81.601458 80.4) (width 0.4) (layer B.Cu) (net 15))
 (via (at 81.45 81.4) (size 0.8) (drill 0.4) (layers F.Cu B.Cu) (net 16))
 (segment (start 86.940001 83.629999) (end 87.79 82.78) (width 0.4) (layer B.Cu) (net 16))
 (segment (start 84.080001 84.030001) (end 86.539999 84.030001) (width 0.4) (layer B.Cu) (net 16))
 (segment (start 86.539999 84.030001) (end 86.940001 83.629999) (width 0.4) (layer B.Cu) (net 16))
 (segment (start 81.45 81.4) (end 84.080001 84.030001) (width 0.4) (layer B.Cu) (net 16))
 (segment (start 81.425 81.375) (end 81.45 81.4) (width 0.4) (layer F.Cu) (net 16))
 (segment (start 78.05 81.375) (end 81.425 81.375) (width 0.4) (layer F.Cu) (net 16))
 (segment (start 78 81.4) (end 81.45 81.4) (width 0.4) (layer B.Cu) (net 16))
 (via (at 81.45 69.4) (size 0.8) (drill 0.4) (layers F.Cu B.Cu) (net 4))
 (segment (start 86.940001 68.389999) (end 87.79 67.54) (width 0.4) (layer B.Cu) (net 4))
 (segment (start 86.500001 68.829999) (end 86.940001 68.389999) (width 0.4) (layer B.Cu) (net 4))
 (segment (start 82.020001 68.829999) (end 86.500001 68.829999) (width 0.4) (layer B.Cu) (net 4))
 (segment (start 81.45 69.4) (end 82.020001 68.829999) (width 0.4) (layer B.Cu) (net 4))
 (segment (start 81.425 69.375) (end 81.45 69.4) (width 0.4) (layer F.Cu) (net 4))
 (segment (start 78.05 69.375) (end 81.425 69.375) (width 0.4) (layer F.Cu) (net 4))
 (segment (start 78 69.4) (end 81.45 69.4) (width 0.4) (layer B.Cu) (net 4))
 (segment (start 84.955 70.375) (end 85.25 70.08) (width 0.4) (layer F.Cu) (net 5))
 (segment (start 78.05 70.375) (end 84.955 70.375) (width 0.4) (layer F.Cu) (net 5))
 (segment (start 84.93 70.4) (end 85.25 70.08) (width 0.4) (layer B.Cu) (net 5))
 (segment (start 78 70.4) (end 84.93 70.4) (width 0.4) (layer B.Cu) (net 5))
 (via (at 81.45 71.4) (size 0.8) (drill 0.4) (layers F.Cu B.Cu) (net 6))
 (segment (start 86.940001 70.929999) (end 87.79 70.08) (width 0.4) (layer B.Cu) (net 6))
 (segment (start 86.500001 71.369999) (end 86.940001 70.929999) (width 0.4) (layer B.Cu) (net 6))
 (segment (start 84.649999 71.369999) (end 86.500001 71.369999) (width 0.4) (layer B.Cu) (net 6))
 (segment (start 84.619998 71.4) (end 84.649999 71.369999) (width 0.4) (layer B.Cu) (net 6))
 (segment (start 81.45 71.4) (end 84.619998 71.4) (width 0.4) (layer B.Cu) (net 6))
 (segment (start 81.425 71.375) (end 81.45 71.4) (width 0.4) (layer F.Cu) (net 6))
 (segment (start 78.05 71.375) (end 81.425 71.375) (width 0.4) (layer F.Cu) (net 6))
 (segment (start 78 71.4) (end 81.45 71.4) (width 0.4) (layer B.Cu) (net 6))
 (segment (start 85.005 72.375) (end 85.25 72.62) (width 0.4) (layer F.Cu) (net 7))
 (segment (start 78.05 72.375) (end 85.005 72.375) (width 0.4) (layer F.Cu) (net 7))
 (segment (start 85.03 72.4) (end 85.25 72.62) (width 0.4) (layer B.Cu) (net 7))
 (segment (start 78 72.4) (end 85.03 72.4) (width 0.4) (layer B.Cu) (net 7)))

